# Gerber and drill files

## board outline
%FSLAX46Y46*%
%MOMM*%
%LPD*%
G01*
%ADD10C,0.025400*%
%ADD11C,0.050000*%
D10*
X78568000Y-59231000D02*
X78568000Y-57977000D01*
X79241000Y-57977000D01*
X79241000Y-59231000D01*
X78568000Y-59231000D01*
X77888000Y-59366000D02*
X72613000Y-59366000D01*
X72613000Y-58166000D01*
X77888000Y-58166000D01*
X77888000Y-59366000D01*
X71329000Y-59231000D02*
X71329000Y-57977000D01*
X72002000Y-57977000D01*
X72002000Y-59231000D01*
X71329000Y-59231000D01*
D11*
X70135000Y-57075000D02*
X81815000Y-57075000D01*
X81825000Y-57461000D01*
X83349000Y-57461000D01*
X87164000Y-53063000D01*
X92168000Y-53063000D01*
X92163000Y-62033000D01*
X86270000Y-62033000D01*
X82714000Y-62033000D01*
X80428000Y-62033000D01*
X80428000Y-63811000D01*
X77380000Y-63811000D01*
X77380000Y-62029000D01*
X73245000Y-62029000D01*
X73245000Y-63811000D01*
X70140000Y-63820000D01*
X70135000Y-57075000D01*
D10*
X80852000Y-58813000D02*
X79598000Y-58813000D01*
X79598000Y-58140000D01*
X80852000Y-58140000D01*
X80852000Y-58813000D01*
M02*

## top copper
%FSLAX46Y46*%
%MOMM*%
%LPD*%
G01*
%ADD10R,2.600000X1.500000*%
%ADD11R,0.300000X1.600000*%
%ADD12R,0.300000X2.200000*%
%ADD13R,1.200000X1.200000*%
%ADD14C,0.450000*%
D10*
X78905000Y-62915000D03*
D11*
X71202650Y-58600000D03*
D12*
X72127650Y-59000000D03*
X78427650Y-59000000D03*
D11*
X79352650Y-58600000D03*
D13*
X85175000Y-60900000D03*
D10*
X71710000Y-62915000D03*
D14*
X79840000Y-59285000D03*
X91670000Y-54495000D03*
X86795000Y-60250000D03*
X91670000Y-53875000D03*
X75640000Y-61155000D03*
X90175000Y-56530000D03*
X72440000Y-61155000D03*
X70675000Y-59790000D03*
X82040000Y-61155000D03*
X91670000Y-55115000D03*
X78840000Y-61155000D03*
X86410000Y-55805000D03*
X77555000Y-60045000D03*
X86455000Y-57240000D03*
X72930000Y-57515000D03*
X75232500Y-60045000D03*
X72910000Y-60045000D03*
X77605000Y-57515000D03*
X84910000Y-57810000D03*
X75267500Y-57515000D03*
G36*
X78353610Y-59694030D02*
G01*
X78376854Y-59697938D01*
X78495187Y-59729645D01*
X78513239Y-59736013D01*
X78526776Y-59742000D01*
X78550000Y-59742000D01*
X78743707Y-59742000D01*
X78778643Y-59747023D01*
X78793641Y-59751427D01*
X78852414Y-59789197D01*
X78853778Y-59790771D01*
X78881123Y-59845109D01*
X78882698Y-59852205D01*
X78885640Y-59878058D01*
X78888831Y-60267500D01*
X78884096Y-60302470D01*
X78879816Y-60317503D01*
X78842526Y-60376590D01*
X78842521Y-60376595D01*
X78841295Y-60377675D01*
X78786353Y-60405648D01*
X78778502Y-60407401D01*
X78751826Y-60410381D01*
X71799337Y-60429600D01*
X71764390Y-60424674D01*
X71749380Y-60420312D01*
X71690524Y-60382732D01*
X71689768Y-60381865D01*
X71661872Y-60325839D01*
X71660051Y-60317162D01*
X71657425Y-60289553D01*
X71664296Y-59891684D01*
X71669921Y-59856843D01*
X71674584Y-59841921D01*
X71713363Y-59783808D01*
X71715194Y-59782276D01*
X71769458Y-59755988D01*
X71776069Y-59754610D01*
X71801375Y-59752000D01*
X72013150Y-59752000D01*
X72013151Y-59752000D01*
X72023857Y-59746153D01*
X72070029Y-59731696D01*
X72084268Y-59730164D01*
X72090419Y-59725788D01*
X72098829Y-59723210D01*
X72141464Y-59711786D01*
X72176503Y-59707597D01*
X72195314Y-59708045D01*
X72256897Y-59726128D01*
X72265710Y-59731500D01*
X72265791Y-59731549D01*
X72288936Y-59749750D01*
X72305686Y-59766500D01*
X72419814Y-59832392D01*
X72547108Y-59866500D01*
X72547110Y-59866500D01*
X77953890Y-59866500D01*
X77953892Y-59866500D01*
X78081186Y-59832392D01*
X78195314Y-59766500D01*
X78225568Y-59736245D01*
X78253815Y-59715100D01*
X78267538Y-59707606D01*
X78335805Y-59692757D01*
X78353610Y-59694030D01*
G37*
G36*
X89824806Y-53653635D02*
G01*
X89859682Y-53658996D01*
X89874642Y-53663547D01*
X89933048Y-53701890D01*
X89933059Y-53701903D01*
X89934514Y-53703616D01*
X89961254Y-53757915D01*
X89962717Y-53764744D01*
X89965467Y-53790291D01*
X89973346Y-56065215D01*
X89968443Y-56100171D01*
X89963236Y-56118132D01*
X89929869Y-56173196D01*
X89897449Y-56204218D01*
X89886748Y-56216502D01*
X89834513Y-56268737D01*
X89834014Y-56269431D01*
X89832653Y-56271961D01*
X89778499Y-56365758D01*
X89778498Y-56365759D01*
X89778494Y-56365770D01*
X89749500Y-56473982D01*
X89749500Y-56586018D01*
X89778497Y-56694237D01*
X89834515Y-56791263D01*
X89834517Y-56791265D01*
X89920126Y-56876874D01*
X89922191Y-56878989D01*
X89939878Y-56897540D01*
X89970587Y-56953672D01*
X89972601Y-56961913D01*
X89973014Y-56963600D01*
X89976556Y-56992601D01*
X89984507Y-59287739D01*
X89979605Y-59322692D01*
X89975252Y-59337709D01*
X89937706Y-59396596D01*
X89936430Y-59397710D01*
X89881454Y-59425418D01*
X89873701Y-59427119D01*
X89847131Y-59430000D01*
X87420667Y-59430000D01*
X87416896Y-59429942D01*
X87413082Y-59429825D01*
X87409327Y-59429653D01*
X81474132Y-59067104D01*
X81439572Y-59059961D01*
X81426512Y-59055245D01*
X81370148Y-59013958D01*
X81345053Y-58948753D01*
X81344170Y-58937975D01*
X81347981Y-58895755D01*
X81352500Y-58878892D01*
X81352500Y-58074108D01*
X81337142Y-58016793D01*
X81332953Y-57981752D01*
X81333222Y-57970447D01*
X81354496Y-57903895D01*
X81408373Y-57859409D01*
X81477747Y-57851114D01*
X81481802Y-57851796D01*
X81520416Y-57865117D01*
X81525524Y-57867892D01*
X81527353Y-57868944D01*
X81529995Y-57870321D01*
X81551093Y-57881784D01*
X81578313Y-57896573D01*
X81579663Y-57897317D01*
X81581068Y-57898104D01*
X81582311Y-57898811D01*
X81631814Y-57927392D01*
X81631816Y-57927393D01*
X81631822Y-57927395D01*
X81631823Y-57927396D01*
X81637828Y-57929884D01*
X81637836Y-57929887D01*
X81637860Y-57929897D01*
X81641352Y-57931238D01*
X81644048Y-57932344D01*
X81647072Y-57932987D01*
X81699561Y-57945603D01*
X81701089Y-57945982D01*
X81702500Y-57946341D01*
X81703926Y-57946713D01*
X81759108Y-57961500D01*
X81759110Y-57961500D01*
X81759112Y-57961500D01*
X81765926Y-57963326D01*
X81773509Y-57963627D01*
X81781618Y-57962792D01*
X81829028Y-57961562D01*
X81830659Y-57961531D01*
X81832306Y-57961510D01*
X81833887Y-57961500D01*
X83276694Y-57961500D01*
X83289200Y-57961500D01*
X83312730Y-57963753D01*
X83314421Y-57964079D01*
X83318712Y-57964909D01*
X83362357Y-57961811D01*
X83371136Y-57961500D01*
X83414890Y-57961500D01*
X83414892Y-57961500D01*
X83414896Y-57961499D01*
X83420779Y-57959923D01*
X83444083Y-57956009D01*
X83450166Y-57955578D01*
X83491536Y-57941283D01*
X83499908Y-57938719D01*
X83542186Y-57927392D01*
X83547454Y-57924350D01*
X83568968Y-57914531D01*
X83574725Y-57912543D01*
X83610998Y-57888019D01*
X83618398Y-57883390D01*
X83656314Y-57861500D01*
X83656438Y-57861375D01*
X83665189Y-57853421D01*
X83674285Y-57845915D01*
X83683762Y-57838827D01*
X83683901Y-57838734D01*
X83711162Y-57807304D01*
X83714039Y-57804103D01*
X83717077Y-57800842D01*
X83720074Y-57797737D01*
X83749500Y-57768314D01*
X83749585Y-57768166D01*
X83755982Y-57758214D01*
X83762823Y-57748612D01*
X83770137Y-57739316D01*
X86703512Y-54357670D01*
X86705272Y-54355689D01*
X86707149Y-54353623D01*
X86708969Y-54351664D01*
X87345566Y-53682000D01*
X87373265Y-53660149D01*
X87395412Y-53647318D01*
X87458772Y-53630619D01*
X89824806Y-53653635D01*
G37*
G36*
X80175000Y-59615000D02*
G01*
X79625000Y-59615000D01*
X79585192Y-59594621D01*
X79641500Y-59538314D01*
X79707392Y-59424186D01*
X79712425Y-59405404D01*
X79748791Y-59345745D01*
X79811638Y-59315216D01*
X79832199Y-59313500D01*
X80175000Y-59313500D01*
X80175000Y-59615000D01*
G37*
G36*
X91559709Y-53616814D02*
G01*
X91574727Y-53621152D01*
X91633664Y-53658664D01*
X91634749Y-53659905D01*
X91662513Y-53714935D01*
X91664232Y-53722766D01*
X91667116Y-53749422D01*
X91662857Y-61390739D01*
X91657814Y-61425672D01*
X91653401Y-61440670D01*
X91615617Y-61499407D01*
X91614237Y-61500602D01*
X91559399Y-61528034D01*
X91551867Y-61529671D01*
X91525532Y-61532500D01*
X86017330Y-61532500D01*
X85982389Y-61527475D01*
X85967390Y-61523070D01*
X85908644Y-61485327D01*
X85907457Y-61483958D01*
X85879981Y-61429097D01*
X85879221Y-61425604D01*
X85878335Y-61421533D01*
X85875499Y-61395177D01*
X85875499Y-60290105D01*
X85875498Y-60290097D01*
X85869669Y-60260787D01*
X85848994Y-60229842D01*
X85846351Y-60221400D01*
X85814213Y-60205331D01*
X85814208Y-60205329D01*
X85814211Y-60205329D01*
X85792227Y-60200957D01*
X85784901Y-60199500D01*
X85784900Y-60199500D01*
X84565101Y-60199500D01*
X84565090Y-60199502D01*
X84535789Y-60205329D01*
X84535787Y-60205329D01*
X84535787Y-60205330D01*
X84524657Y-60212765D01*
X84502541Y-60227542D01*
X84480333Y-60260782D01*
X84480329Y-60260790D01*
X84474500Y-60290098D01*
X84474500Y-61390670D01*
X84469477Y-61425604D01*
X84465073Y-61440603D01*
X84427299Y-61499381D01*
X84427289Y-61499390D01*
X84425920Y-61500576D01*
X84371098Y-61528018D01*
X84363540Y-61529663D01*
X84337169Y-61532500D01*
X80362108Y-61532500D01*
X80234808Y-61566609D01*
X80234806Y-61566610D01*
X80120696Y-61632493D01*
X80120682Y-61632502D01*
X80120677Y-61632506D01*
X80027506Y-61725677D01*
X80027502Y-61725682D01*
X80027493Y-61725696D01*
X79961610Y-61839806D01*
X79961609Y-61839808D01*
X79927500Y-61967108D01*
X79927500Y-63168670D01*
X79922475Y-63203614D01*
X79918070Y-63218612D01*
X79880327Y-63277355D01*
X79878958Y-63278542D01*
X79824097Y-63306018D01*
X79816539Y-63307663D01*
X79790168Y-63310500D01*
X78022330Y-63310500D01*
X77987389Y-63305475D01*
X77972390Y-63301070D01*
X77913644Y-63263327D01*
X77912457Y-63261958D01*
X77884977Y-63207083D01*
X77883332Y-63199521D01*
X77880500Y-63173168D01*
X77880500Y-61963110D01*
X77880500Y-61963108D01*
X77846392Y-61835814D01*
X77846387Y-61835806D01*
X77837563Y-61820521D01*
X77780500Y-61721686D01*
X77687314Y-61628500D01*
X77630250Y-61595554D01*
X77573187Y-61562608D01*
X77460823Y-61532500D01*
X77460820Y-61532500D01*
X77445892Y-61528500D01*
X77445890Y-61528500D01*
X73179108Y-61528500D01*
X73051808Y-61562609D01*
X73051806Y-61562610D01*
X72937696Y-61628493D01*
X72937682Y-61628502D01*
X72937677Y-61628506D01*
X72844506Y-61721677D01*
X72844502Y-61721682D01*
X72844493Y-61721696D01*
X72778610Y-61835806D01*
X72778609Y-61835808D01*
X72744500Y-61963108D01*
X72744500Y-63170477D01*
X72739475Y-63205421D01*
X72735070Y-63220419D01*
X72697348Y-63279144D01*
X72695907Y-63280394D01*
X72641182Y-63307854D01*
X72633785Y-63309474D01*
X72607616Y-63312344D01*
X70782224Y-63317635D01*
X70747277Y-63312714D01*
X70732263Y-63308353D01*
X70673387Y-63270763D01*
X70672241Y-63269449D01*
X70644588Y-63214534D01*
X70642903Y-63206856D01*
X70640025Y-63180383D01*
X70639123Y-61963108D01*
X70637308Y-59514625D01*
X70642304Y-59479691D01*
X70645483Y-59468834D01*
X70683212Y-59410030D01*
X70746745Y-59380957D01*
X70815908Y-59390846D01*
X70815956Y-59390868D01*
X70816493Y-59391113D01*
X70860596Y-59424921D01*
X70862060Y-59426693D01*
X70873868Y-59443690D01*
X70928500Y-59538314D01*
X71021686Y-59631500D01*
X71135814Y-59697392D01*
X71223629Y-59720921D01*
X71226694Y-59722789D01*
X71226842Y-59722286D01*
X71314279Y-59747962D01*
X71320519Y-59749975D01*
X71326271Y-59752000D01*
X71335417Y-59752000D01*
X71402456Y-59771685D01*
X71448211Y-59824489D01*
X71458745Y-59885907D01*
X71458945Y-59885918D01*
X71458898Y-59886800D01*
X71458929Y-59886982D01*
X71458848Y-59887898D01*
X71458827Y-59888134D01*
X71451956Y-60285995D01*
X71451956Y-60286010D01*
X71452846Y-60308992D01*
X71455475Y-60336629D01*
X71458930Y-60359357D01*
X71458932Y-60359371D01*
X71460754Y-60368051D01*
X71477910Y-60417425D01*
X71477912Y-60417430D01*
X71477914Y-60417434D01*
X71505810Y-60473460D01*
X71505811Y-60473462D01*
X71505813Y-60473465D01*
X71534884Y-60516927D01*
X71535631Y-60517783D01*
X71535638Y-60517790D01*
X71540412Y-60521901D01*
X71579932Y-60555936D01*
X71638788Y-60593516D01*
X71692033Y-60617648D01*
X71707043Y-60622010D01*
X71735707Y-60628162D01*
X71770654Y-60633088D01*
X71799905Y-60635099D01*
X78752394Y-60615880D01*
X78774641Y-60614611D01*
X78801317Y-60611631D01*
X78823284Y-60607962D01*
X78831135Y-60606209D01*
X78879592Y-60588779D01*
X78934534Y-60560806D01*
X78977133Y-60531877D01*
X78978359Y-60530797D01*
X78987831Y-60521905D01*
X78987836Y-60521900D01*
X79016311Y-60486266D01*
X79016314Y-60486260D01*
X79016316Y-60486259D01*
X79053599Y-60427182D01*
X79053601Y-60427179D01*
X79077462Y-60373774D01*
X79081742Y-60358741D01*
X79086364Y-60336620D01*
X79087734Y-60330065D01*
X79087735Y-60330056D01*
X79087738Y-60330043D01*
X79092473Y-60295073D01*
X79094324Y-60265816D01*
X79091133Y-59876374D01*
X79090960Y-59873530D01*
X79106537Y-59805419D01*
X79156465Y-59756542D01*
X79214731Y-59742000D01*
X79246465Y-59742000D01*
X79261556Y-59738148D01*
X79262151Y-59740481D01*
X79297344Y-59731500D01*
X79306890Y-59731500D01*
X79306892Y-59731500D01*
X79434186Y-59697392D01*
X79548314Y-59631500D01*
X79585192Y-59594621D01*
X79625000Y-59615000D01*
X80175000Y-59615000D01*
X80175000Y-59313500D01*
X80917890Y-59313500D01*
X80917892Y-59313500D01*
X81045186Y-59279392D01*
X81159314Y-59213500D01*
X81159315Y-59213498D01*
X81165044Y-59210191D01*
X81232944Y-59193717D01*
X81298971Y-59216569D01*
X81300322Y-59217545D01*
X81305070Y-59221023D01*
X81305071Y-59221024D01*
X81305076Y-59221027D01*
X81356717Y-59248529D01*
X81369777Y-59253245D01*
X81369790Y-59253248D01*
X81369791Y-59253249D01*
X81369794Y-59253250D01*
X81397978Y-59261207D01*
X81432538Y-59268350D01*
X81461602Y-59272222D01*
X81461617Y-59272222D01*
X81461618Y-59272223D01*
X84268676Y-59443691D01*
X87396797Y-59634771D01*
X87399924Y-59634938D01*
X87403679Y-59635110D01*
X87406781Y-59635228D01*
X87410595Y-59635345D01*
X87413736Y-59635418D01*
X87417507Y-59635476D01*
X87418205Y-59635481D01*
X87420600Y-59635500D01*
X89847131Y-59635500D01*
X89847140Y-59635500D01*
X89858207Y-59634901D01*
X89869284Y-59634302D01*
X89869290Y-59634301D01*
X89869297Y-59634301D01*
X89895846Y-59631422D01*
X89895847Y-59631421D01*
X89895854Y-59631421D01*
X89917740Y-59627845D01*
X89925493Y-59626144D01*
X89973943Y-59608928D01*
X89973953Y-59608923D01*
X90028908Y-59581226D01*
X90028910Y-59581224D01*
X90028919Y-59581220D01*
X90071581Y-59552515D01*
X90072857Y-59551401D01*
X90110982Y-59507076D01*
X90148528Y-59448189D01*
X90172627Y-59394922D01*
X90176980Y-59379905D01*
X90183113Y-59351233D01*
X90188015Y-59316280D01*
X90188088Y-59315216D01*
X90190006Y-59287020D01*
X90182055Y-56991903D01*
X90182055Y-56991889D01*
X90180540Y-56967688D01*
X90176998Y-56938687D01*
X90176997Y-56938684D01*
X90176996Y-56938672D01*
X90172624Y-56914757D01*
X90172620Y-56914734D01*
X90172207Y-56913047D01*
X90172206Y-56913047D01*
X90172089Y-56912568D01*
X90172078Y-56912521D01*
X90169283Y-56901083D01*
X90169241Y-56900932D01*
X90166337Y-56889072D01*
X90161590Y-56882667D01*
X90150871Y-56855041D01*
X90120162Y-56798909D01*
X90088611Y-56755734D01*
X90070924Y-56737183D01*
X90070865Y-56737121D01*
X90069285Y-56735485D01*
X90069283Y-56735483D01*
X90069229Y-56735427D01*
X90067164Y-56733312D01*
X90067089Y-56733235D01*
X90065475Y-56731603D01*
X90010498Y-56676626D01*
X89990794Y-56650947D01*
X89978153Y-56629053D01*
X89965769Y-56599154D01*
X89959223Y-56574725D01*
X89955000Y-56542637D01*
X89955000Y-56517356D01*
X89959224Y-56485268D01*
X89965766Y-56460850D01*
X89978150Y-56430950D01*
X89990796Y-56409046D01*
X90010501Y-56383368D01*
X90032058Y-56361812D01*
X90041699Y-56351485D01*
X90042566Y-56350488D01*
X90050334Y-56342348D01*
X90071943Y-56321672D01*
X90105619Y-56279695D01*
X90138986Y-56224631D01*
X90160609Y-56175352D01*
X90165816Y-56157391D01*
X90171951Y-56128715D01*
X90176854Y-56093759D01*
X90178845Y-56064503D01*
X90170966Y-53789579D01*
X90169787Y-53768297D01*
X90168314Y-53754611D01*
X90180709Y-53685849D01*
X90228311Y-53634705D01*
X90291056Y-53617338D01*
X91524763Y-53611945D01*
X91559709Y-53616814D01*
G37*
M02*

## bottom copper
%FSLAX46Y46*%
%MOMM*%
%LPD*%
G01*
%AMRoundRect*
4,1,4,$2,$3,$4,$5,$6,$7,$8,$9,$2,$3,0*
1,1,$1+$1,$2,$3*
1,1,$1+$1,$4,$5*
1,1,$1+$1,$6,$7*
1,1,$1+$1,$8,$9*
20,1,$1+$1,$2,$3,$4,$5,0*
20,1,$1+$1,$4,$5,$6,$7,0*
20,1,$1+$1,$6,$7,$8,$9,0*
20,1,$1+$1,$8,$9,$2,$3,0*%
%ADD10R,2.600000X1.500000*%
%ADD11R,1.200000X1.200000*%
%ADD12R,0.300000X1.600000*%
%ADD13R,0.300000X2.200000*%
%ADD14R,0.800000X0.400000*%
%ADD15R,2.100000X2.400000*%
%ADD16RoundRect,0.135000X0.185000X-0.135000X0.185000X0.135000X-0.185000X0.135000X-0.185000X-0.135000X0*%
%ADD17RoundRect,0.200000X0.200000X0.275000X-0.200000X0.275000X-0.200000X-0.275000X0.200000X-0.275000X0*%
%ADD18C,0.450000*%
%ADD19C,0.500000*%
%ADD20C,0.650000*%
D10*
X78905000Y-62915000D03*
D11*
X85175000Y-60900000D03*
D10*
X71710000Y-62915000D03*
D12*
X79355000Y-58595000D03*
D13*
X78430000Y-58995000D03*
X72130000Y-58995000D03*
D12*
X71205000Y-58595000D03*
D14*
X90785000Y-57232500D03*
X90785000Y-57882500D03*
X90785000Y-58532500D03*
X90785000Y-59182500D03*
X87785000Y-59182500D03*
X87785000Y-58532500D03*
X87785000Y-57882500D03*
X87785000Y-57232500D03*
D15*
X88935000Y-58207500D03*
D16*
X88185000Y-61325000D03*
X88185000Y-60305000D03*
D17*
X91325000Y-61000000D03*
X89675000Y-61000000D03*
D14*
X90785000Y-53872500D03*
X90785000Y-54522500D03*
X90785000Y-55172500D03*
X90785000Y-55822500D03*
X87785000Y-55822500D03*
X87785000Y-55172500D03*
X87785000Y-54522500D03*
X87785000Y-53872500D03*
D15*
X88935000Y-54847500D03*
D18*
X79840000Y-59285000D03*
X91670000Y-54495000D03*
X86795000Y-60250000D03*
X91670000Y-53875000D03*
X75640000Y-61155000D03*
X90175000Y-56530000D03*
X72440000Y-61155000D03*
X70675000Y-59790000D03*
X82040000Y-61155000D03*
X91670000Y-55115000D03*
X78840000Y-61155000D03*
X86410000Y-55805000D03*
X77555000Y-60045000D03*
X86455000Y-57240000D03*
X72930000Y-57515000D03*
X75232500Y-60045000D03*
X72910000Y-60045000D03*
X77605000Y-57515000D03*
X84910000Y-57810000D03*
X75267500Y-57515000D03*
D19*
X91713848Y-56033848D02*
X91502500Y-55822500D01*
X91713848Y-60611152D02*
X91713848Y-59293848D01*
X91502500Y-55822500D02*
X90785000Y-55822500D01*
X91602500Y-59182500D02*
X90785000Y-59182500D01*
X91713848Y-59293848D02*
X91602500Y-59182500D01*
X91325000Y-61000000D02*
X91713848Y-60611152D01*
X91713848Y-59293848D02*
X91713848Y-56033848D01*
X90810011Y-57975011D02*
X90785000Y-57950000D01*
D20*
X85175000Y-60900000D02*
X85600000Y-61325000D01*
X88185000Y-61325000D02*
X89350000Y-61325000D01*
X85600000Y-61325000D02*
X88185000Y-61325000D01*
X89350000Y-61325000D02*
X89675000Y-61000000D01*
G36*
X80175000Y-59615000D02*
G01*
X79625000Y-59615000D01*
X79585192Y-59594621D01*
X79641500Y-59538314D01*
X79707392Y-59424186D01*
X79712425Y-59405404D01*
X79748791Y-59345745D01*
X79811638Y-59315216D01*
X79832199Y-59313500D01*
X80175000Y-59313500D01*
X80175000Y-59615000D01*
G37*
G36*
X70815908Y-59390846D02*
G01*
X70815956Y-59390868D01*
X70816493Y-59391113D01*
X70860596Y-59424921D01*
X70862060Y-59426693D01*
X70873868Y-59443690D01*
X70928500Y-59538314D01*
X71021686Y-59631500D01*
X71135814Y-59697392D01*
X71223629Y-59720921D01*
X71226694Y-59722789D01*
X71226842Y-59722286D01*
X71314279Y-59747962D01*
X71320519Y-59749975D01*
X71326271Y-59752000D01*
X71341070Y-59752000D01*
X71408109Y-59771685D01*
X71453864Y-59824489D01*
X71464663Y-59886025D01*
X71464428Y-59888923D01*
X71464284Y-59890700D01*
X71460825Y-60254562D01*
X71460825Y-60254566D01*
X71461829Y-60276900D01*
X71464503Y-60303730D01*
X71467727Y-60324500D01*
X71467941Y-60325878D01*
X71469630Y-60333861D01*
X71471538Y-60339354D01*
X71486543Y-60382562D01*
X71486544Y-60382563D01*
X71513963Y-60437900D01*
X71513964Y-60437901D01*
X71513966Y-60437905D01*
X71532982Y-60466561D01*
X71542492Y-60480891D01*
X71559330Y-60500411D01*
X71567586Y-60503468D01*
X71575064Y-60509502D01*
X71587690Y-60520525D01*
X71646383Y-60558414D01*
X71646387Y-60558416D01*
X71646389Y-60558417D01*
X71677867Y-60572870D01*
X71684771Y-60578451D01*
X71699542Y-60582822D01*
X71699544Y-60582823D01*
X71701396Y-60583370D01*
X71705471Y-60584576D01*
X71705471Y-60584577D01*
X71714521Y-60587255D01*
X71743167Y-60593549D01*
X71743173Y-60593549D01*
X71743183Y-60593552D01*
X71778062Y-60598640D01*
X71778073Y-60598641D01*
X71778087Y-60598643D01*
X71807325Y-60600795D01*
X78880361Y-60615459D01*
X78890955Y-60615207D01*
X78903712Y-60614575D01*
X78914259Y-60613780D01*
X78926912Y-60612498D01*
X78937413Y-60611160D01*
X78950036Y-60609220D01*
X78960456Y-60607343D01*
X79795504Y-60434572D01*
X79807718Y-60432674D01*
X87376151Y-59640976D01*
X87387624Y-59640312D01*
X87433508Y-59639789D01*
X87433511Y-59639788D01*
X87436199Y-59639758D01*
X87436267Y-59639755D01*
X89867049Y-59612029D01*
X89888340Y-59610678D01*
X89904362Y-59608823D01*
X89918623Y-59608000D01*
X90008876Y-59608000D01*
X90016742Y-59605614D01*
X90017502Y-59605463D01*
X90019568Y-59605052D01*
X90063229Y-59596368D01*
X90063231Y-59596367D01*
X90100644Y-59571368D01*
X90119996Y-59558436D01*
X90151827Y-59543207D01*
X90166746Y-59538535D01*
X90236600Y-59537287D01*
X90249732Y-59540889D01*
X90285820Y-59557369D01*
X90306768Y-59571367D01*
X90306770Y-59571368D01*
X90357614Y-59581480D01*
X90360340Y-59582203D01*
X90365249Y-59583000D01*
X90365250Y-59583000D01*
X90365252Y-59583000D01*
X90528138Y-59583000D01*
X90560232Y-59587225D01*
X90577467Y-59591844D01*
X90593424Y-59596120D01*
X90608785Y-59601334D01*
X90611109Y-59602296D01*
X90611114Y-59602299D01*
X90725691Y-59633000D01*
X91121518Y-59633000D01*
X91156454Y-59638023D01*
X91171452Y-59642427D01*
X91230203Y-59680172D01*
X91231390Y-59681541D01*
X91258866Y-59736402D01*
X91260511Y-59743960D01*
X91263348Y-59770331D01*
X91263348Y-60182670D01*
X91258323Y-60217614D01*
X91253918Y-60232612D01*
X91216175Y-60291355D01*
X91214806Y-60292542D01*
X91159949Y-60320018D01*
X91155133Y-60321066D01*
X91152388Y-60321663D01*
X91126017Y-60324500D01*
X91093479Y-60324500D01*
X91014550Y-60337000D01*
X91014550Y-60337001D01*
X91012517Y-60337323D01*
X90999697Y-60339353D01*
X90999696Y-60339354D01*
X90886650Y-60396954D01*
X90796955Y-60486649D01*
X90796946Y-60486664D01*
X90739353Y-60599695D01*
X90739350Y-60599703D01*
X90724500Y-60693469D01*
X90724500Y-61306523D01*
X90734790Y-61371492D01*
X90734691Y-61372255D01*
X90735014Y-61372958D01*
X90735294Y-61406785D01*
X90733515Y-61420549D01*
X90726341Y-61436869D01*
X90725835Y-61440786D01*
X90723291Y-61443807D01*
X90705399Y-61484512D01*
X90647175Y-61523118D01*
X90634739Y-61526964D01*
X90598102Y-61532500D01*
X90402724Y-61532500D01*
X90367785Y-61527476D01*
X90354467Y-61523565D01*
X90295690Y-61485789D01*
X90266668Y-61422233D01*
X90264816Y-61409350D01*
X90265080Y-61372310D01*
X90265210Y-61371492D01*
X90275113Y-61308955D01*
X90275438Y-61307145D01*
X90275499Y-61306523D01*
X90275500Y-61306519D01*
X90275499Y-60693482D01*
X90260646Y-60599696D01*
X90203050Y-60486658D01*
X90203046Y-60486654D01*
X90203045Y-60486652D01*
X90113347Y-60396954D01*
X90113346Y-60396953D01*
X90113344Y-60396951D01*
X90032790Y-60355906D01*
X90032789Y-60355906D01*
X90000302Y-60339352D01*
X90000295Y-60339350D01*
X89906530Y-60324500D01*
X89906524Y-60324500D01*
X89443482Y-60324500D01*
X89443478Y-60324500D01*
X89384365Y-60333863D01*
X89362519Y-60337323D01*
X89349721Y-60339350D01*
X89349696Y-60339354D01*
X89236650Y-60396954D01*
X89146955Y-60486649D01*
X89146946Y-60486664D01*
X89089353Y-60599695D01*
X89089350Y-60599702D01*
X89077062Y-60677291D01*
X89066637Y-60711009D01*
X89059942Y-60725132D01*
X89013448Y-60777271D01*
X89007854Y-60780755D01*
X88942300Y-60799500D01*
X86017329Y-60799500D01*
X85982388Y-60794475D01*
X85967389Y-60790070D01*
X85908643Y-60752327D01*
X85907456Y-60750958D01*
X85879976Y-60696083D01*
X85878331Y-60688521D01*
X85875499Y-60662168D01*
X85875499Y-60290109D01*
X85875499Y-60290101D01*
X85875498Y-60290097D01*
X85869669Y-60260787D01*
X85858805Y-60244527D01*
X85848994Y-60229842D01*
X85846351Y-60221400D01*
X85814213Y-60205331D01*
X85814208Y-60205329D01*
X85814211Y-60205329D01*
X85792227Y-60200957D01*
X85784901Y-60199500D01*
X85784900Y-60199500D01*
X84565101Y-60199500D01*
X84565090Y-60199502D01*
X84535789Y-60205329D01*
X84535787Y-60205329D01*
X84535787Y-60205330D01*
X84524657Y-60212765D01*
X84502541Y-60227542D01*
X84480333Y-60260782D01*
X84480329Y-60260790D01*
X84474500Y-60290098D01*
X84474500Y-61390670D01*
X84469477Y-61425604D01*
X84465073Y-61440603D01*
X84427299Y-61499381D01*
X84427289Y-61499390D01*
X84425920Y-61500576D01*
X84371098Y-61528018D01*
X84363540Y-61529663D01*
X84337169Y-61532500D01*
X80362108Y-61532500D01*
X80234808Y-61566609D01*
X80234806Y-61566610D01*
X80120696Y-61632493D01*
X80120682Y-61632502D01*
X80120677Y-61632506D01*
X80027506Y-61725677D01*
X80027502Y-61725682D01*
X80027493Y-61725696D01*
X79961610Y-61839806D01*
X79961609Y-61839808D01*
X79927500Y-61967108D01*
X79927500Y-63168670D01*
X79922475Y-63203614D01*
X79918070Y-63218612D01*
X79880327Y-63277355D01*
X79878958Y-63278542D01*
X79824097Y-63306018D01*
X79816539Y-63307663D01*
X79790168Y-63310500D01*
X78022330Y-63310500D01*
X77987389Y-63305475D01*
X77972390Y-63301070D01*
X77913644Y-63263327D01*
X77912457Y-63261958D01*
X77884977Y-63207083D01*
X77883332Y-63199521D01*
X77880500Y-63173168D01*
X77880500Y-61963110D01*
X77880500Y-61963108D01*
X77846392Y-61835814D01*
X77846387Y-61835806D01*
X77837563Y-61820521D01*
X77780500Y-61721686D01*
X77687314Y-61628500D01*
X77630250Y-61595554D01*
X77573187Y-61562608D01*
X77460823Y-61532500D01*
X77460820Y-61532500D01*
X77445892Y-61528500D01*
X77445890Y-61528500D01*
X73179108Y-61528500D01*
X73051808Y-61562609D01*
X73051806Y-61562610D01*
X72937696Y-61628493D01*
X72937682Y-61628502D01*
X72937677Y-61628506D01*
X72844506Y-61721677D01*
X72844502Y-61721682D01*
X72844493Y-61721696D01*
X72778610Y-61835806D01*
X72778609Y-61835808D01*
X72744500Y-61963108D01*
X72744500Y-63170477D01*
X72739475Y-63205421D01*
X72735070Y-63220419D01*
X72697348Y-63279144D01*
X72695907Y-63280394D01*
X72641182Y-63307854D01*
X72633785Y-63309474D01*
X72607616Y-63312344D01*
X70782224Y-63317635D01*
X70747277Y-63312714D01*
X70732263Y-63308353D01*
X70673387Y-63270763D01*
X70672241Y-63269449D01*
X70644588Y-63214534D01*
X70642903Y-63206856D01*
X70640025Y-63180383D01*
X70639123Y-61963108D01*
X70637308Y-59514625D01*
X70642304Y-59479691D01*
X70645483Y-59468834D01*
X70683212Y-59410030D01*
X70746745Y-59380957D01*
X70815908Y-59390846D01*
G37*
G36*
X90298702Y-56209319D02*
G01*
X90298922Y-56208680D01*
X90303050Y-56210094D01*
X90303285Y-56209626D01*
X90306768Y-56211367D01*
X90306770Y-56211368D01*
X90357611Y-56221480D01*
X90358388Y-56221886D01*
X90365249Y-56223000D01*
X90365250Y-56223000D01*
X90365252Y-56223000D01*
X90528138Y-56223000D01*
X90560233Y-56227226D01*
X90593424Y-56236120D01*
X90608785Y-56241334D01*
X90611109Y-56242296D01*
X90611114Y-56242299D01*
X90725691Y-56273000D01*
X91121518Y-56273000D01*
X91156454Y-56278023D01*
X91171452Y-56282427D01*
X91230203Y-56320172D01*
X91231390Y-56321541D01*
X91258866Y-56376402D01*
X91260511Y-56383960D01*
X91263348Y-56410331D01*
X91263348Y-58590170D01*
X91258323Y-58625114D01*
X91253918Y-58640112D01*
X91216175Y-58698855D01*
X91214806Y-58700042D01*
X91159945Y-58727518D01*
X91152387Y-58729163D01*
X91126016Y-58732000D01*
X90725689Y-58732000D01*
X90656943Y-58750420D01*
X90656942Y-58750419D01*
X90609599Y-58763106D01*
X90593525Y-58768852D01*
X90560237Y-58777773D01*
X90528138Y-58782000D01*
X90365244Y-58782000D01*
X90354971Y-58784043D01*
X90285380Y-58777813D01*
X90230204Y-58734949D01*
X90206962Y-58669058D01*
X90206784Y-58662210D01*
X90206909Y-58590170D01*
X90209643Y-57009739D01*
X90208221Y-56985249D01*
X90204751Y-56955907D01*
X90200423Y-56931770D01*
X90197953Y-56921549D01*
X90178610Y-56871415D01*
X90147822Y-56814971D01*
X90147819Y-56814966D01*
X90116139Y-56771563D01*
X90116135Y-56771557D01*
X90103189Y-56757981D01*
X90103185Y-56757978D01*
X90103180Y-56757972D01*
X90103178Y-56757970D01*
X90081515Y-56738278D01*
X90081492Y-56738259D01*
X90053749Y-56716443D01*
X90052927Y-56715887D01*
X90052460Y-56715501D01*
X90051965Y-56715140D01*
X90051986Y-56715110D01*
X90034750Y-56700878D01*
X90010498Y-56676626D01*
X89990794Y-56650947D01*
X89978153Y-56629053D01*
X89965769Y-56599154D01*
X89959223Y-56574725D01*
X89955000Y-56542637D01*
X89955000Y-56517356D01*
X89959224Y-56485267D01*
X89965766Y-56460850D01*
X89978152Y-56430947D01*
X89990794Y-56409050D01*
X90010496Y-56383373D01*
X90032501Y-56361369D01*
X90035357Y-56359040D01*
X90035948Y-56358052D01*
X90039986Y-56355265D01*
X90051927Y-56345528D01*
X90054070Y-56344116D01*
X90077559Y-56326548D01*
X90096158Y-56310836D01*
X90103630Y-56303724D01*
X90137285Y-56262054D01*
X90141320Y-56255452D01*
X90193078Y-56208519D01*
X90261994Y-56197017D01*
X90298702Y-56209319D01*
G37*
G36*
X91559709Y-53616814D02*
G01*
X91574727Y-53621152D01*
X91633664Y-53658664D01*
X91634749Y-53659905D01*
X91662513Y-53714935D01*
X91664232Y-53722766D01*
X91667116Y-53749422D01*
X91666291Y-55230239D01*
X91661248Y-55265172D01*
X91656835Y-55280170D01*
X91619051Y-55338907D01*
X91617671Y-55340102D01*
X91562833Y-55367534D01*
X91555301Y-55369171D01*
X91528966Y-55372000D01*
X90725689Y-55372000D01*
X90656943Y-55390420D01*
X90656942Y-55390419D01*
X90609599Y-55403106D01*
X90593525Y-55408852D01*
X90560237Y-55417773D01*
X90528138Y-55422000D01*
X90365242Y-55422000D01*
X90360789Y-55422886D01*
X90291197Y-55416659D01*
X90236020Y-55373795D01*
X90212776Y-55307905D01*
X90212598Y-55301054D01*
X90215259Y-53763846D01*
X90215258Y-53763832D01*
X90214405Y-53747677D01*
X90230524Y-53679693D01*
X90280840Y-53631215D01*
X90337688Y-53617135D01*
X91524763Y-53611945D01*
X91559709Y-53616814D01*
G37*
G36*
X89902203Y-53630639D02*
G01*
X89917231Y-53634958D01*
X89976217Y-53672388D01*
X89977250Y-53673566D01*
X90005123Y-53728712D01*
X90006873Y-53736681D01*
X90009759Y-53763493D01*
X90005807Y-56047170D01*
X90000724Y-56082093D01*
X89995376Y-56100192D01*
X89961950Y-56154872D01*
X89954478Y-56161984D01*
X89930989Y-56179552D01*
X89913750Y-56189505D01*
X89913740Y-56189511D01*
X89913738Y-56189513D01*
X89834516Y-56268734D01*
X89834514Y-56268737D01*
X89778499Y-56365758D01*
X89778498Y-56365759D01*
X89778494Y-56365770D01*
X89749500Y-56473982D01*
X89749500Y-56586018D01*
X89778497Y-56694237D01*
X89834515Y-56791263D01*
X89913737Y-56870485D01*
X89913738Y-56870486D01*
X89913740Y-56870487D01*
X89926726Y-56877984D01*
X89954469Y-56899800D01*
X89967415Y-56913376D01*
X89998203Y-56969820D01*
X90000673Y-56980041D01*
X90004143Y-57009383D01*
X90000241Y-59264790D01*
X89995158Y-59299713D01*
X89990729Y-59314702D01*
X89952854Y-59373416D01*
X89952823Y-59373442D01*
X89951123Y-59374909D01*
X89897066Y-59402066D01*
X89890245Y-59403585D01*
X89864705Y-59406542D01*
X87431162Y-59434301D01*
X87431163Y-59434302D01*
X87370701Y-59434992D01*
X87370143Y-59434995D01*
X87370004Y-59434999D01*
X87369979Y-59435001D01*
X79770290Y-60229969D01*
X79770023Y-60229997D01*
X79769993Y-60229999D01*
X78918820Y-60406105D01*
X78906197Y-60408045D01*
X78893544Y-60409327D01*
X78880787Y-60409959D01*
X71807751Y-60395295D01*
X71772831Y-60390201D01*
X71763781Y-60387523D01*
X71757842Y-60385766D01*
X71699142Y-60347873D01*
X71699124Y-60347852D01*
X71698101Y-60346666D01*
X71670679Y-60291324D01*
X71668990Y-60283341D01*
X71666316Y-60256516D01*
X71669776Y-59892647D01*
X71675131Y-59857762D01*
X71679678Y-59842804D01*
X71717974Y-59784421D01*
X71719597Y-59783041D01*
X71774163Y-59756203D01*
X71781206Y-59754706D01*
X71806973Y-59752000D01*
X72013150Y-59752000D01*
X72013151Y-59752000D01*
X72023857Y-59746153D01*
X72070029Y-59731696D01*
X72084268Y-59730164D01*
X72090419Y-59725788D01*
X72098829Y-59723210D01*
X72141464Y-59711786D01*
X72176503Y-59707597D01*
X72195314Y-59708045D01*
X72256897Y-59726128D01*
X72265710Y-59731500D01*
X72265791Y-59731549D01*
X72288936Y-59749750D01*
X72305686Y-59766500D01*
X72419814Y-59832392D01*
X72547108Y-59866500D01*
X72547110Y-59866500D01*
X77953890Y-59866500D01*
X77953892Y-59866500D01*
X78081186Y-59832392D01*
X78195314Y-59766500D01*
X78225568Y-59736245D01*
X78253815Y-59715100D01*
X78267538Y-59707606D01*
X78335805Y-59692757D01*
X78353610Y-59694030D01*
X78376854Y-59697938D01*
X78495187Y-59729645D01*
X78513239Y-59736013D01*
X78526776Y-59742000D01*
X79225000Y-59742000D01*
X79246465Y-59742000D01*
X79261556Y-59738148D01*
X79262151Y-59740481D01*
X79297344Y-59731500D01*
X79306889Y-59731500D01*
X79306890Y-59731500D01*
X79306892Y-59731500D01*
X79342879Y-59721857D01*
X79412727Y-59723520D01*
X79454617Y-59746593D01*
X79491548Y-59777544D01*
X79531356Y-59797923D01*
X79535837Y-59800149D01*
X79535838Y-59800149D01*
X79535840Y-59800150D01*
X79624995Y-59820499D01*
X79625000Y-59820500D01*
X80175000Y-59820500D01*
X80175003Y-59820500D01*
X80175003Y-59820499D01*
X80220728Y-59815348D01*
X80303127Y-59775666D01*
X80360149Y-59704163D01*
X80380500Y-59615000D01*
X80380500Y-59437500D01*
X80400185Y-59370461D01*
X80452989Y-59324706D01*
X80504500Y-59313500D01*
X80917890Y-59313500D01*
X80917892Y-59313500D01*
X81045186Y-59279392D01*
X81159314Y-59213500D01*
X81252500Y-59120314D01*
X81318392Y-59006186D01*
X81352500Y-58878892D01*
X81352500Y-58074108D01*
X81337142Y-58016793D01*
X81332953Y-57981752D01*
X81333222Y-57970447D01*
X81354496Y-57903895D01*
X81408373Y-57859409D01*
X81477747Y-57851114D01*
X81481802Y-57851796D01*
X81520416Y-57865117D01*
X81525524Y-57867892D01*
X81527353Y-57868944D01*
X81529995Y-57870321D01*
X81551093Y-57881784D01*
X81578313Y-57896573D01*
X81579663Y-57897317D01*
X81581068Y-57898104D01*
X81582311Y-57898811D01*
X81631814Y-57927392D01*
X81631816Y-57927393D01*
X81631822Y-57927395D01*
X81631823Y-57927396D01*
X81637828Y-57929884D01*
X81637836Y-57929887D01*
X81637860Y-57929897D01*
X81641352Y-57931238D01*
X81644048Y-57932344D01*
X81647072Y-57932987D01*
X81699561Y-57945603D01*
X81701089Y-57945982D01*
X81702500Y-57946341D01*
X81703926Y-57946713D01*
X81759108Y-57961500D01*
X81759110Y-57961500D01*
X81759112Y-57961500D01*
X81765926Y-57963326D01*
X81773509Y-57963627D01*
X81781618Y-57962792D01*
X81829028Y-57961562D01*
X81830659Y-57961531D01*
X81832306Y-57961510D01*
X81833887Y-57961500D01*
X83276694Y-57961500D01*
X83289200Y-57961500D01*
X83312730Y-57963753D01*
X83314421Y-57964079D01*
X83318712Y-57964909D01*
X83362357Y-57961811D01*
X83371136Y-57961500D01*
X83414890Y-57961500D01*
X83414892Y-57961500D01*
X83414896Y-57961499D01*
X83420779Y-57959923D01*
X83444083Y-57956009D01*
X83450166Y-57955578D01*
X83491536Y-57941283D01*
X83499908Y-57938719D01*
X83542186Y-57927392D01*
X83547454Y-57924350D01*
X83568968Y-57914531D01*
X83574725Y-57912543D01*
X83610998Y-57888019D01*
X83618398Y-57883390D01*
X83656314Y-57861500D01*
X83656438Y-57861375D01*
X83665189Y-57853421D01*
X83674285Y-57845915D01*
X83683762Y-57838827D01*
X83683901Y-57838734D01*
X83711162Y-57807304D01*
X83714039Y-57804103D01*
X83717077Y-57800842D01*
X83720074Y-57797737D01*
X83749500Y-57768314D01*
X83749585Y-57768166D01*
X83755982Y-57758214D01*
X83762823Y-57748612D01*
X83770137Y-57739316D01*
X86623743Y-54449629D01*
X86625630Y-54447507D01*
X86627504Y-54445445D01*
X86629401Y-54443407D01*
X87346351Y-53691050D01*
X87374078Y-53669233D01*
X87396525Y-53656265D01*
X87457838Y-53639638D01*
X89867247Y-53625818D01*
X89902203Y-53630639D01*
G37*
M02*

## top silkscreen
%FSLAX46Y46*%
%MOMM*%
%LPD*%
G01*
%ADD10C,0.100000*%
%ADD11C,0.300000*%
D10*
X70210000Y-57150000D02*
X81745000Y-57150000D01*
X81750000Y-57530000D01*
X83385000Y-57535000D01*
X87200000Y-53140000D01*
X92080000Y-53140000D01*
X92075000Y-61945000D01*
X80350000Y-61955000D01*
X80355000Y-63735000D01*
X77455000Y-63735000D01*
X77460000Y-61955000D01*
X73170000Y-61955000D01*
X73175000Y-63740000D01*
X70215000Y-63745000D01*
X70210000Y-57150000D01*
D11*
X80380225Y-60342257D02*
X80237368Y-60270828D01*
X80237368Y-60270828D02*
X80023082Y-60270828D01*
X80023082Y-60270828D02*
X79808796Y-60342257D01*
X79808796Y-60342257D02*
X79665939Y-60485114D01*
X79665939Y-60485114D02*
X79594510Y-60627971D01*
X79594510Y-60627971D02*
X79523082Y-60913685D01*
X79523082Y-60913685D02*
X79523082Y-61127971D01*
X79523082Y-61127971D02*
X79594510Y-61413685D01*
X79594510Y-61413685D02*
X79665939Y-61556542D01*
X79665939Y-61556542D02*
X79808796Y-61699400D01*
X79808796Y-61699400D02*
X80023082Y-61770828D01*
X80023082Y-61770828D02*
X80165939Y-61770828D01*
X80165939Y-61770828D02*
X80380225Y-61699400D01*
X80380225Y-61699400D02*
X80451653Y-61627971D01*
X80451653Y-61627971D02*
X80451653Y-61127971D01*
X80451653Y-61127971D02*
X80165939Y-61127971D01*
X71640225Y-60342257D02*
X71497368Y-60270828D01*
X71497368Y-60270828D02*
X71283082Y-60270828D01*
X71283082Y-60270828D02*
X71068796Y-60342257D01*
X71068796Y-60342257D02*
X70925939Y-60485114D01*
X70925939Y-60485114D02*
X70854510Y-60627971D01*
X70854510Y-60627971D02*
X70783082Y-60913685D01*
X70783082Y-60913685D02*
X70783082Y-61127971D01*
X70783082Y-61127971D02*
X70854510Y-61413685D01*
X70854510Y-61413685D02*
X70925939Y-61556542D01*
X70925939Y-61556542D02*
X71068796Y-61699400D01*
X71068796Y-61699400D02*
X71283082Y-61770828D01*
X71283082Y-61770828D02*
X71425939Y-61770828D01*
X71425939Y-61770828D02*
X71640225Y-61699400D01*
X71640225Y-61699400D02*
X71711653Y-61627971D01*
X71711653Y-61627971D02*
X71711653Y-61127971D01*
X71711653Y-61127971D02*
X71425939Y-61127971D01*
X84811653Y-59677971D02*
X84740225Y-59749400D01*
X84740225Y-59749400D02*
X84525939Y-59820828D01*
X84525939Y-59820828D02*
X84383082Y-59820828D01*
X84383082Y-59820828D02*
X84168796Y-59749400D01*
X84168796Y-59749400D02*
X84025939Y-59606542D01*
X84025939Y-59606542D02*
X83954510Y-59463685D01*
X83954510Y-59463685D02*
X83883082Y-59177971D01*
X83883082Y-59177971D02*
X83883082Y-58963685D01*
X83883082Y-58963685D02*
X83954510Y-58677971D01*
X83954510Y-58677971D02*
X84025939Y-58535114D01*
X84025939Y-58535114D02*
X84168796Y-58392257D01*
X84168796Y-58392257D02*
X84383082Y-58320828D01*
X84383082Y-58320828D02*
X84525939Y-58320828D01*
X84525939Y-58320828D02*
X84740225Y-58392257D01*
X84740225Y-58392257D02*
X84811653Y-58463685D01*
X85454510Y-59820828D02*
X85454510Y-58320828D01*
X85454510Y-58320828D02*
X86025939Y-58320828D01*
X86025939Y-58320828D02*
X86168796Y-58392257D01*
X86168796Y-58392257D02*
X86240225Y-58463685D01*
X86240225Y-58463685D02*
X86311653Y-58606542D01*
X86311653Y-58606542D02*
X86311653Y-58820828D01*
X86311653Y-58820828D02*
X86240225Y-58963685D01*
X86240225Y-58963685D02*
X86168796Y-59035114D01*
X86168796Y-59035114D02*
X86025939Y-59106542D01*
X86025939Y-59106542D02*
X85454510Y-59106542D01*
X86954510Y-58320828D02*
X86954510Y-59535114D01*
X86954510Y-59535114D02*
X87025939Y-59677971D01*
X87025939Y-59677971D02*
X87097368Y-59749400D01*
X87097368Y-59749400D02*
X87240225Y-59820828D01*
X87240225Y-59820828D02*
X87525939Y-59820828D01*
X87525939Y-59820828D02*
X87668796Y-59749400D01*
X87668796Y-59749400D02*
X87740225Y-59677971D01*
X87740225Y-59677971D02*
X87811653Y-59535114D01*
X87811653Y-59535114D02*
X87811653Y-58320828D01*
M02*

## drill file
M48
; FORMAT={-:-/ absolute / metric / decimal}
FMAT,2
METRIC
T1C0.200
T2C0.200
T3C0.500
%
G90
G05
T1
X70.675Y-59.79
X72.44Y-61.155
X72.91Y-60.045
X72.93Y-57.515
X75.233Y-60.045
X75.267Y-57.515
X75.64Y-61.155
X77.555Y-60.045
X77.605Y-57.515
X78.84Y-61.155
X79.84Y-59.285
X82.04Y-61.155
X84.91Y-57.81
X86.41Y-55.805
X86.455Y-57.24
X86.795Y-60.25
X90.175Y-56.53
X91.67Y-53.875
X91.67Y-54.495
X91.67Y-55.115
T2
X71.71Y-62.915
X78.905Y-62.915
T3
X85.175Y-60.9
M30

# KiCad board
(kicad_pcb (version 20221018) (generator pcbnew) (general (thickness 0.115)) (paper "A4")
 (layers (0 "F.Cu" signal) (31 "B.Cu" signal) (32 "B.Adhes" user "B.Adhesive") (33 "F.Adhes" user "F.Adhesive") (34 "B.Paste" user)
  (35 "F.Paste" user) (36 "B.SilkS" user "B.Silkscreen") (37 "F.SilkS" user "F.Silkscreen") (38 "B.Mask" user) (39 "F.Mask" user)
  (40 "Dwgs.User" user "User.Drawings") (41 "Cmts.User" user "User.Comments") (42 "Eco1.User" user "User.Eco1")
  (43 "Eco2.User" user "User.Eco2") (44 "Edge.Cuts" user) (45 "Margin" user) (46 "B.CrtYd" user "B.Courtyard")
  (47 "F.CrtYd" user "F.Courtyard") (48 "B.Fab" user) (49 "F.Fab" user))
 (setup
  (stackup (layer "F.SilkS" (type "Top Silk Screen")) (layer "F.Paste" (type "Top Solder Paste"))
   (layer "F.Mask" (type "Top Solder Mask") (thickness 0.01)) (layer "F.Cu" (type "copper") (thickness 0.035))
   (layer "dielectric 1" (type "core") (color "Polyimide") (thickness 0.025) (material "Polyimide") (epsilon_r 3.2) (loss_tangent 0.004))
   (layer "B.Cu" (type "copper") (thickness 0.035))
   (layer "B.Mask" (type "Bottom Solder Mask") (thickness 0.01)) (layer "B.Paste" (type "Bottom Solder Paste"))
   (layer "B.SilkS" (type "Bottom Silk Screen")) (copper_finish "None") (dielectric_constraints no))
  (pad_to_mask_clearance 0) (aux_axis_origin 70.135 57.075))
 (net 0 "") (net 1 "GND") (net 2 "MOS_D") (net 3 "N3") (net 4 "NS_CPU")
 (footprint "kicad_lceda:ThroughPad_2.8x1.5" (layer "F.Cu") (at 78.905 62.915)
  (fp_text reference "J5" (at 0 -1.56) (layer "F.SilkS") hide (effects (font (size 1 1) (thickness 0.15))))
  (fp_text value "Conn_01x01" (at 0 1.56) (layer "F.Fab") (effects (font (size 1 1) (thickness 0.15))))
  (pad "1" thru_hole rect (at 0 0) (size 2.6 1.5) (drill 0.2) (layers "*.Cu" "*.Mask") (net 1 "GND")))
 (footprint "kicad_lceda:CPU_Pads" (layer "F.Cu") (at 75.07765 58.6)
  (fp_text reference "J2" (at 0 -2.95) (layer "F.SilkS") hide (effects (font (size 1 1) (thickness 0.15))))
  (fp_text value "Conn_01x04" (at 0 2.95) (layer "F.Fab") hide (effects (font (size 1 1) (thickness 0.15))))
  (pad "1" smd rect (at -3.875 0) (size 0.3 1.6) (layers "F.Cu" "F.Mask") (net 1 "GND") (zone_connect 2))
  (pad "2" smd rect (at -2.95 1) (size 0.3 2.2) (drill (offset 0 -0.6)) (layers "F.Cu" "F.Mask") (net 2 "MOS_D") (clearance 0.3)
   (zone_connect 2))
  (pad "3" smd rect (at 3.35 1) (size 0.3 2.2) (drill (offset 0 -0.6)) (layers "F.Cu" "F.Mask") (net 2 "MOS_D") (clearance 0.3)
   (zone_connect 2))
  (pad "4" smd rect (at 4.275 0) (size 0.3 1.6) (layers "F.Cu" "F.Mask") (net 1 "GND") (zone_connect 2)))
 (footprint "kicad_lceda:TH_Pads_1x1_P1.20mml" (layer "F.Cu") (at 85.175 60.9)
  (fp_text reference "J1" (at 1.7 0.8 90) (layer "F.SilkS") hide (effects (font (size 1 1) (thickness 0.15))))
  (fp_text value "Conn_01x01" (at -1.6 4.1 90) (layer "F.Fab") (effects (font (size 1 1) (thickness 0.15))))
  (pad "1" thru_hole rect (at 0 0) (size 1.2 1.2) (drill 0.5) (layers "*.Cu" "*.Mask") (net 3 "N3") (clearance 0.1) (zone_connect 2)))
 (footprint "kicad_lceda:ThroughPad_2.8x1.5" (layer "F.Cu") (at 71.71 62.915)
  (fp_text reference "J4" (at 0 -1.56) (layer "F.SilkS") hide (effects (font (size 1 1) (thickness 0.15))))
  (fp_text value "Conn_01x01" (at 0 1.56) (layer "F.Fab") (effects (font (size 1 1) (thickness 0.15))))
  (pad "1" thru_hole rect (at 0 0) (size 2.6 1.5) (drill 0.2) (layers "*.Cu" "*.Mask") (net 1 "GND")))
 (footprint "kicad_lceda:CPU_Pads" (layer "B.Cu") (at 75.48 58.595 180)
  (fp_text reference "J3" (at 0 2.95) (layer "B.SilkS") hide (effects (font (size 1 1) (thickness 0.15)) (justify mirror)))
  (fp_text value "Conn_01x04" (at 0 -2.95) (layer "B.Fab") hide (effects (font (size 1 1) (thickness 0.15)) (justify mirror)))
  (pad "1" smd rect (at -3.875 0 180) (size 0.3 1.6) (layers "B.Cu" "B.Mask") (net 1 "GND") (zone_connect 2))
  (pad "2" smd rect (at -2.95 -1 180) (size 0.3 2.2) (drill (offset 0 0.6)) (layers "B.Cu" "B.Mask") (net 2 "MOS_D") (clearance 0.3)
   (zone_connect 2))
  (pad "3" smd rect (at 3.35 -1 180) (size 0.3 2.2) (drill (offset 0 0.6)) (layers "B.Cu" "B.Mask") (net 2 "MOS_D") (clearance 0.3)
   (zone_connect 2))
  (pad "4" smd rect (at 4.275 0 180) (size 0.3 1.6) (layers "B.Cu" "B.Mask") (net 1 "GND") (zone_connect 2)))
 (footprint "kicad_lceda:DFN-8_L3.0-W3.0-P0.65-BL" (layer "B.Cu") (at 89.285 58.2075 -90)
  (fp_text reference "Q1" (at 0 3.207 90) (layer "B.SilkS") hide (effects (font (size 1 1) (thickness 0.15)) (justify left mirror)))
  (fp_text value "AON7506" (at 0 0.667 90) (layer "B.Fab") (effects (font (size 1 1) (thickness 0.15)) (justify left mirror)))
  (pad "1" smd rect (at -0.975 -1.5 90) (size 0.4 0.8) (layers "B.Cu" "B.Paste" "B.Mask") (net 1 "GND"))
  (pad "2" smd rect (at -0.325 -1.5 90) (size 0.4 0.8) (layers "B.Cu" "B.Paste" "B.Mask") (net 1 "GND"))
  (pad "3" smd rect (at 0.325 -1.5 90) (size 0.4 0.8) (layers "B.Cu" "B.Paste" "B.Mask") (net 1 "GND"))
  (pad "4" smd rect (at 0.975 -1.5 90) (size 0.4 0.8) (layers "B.Cu" "B.Paste" "B.Mask") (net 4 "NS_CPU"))
  (pad "5" smd rect (at 0.975 1.5 90) (size 0.4 0.8) (layers "B.Cu" "B.Paste" "B.Mask") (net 2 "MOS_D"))
  (pad "6" smd rect (at 0.325 1.5 90) (size 0.4 0.8) (layers "B.Cu" "B.Paste" "B.Mask") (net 2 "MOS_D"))
  (pad "7" smd rect (at -0.325 1.5 90) (size 0.4 0.8) (layers "B.Cu" "B.Paste" "B.Mask") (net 2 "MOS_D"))
  (pad "8" smd rect (at -0.975 1.5 90) (size 0.4 0.8) (layers "B.Cu" "B.Paste" "B.Mask") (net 2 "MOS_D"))
  (pad "9" smd rect (at 0 0.35 270) (size 2.4 2.1) (layers "B.Cu" "B.Paste" "B.Mask") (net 2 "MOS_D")))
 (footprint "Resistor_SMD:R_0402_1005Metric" (layer "B.Cu") (at 88.185 60.815 90)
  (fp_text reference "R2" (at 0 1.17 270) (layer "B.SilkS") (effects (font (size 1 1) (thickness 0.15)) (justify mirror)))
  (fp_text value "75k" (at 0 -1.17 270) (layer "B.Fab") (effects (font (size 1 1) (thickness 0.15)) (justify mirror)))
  (pad "1" smd roundrect (at -0.51 0 90) (size 0.54 0.64) (layers "B.Cu" "B.Paste" "B.Mask") (roundrect_rratio 0.25) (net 3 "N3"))
  (pad "2" smd roundrect (at 0.51 0 90) (size 0.54 0.64) (layers "B.Cu" "B.Paste" "B.Mask") (roundrect_rratio 0.25) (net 1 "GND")))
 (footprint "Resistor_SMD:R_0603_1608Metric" (layer "B.Cu") (at 90.5 61 180)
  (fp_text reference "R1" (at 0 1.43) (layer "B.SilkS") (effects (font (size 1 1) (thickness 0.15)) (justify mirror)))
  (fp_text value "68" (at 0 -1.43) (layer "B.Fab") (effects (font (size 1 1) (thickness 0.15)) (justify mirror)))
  (pad "1" smd roundrect (at -0.825 0 180) (size 0.8 0.95) (layers "B.Cu" "B.Paste" "B.Mask") (roundrect_rratio 0.25) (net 4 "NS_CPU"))
  (pad "2" smd roundrect (at 0.825 0 180) (size 0.8 0.95) (layers "B.Cu" "B.Paste" "B.Mask") (roundrect_rratio 0.25) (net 3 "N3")))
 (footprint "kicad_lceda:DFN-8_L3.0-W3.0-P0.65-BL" (layer "B.Cu") (at 89.285 54.8475 -90)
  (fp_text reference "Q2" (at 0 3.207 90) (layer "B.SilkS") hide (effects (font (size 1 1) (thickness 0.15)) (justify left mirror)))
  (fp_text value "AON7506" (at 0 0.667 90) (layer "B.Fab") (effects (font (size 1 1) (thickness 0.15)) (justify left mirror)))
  (pad "1" smd rect (at -0.975 -1.5 90) (size 0.4 0.8) (layers "B.Cu" "B.Paste" "B.Mask") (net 1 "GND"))
  (pad "2" smd rect (at -0.325 -1.5 90) (size 0.4 0.8) (layers "B.Cu" "B.Paste" "B.Mask") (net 1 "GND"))
  (pad "3" smd rect (at 0.325 -1.5 90) (size 0.4 0.8) (layers "B.Cu" "B.Paste" "B.Mask") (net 1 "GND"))
  (pad "4" smd rect (at 0.975 -1.5 90) (size 0.4 0.8) (layers "B.Cu" "B.Paste" "B.Mask") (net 4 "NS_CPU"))
  (pad "5" smd rect (at 0.975 1.5 90) (size 0.4 0.8) (layers "B.Cu" "B.Paste" "B.Mask") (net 2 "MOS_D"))
  (pad "6" smd rect (at 0.325 1.5 90) (size 0.4 0.8) (layers "B.Cu" "B.Paste" "B.Mask") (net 2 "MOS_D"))
  (pad "7" smd rect (at -0.325 1.5 90) (size 0.4 0.8) (layers "B.Cu" "B.Paste" "B.Mask") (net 2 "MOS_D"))
  (pad "8" smd rect (at -0.975 1.5 90) (size 0.4 0.8) (layers "B.Cu" "B.Paste" "B.Mask") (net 2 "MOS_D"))
  (pad "9" smd rect (at 0 0.35 270) (size 2.4 2.1) (layers "B.Cu" "B.Paste" "B.Mask") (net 2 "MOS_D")))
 (gr_poly
  (pts (xy 70.21 57.15) (xy 81.745 57.15) (xy 81.75 57.53) (xy 83.385 57.535) (xy 87.2 53.14) (xy 92.08 53.14) (xy 92.075 61.945)
   (xy 80.35 61.955) (xy 80.355 63.735) (xy 77.455 63.735) (xy 77.46 61.955) (xy 73.17 61.955) (xy 73.175 63.74) (xy 70.215 63.745))
  (stroke (width 0.1) (type solid)) (fill none) (layer "F.SilkS"))
 (gr_poly
  (pts (xy 78.568 59.231) (xy 78.568 57.977) (xy 79.241 57.977) (xy 79.241 59.231)) (stroke (width 0.0254) (type solid)) (fill none)
  (layer "Edge.Cuts"))
 (gr_poly
  (pts (xy 77.888 59.366) (xy 72.613 59.366) (xy 72.613 58.166) (xy 77.888 58.166)) (stroke (width 0.0254) (type solid)) (fill none)
  (layer "Edge.Cuts"))
 (gr_poly
  (pts (xy 71.329 59.231) (xy 71.329 57.977) (xy 72.002 57.977) (xy 72.002 59.231)) (stroke (width 0.0254) (type solid)) (fill none)
  (layer "Edge.Cuts"))
 (gr_poly
  (pts (xy 70.135 57.075) (xy 81.815 57.075) (xy 81.825 57.461) (xy 83.349 57.461) (xy 87.164 53.063) (xy 92.168 53.063) (xy 92.163 62.033)
   (xy 86.27 62.033) (xy 82.714 62.033) (xy 80.428 62.033) (xy 80.428 63.811) (xy 77.38 63.811) (xy 77.38 62.029) (xy 73.245 62.029)
   (xy 73.245 63.811) (xy 70.14 63.82))
  (stroke (width 0.05) (type solid)) (fill none) (layer "Edge.Cuts"))
 (gr_poly
  (pts (xy 80.852 58.813) (xy 79.598 58.813) (xy 79.598 58.14) (xy 80.852 58.14)) (stroke (width 0.0254) (type solid)) (fill none)
  (layer "Edge.Cuts"))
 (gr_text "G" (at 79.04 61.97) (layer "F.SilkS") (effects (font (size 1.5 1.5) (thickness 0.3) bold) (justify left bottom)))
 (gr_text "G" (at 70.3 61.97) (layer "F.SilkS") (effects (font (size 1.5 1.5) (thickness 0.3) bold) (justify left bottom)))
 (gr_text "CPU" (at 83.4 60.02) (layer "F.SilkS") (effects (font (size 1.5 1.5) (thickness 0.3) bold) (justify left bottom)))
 (segment (start 91.713848 56.033848) (end 91.5025 55.8225) (width 0.5) (layer "B.Cu") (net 4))
 (segment (start 91.713848 60.611152) (end 91.713848 59.293848) (width 0.5) (layer "B.Cu") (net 4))
 (segment (start 91.5025 55.8225) (end 90.785 55.8225) (width 0.5) (layer "B.Cu") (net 4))
 (segment (start 91.6025 59.1825) (end 90.785 59.1825) (width 0.5) (layer "B.Cu") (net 4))
 (segment (start 91.713848 59.293848) (end 91.6025 59.1825) (width 0.5) (layer "B.Cu") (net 4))
 (segment (start 91.325 61) (end 91.713848 60.611152) (width 0.5) (layer "B.Cu") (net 4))
 (segment (start 91.713848 59.293848) (end 91.713848 56.033848) (width 0.5) (layer "B.Cu") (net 4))
 (via (at 79.84 59.285) (size 0.45) (drill 0.2) (layers "F.Cu" "B.Cu") (free) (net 1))
 (via (at 91.67 54.495) (size 0.45) (drill 0.2) (layers "F.Cu" "B.Cu") (free) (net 1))
 (via (at 86.795 60.25) (size 0.45) (drill 0.2) (layers "F.Cu" "B.Cu") (free) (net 1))
 (via (at 91.67 53.875) (size 0.45) (drill 0.2) (layers "F.Cu" "B.Cu") (free) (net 1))
 (via (at 75.64 61.155) (size 0.45) (drill 0.2) (layers "F.Cu" "B.Cu") (free) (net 1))
 (via (at 90.175 56.53) (size 0.45) (drill 0.2) (layers "F.Cu" "B.Cu") (free) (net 1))
 (via (at 72.44 61.155) (size 0.45) (drill 0.2) (layers "F.Cu" "B.Cu") (free) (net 1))
 (via (at 70.675 59.79) (size 0.45) (drill 0.2) (layers "F.Cu" "B.Cu") (free) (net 1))
 (via (at 82.04 61.155) (size 0.45) (drill 0.2) (layers "F.Cu" "B.Cu") (free) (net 1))
 (via (at 91.67 55.115) (size 0.45) (drill 0.2) (layers "F.Cu" "B.Cu") (free) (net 1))
 (via (at 78.84 61.155) (size 0.45) (drill 0.2) (layers "F.Cu" "B.Cu") (free) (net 1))
 (segment (start 90.810011 57.975011) (end 90.785 57.95) (width 0.5) (layer "B.Cu") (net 1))
 (via (at 86.41 55.805) (size 0.45) (drill 0.2) (layers "F.Cu" "B.Cu") (free) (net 2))
 (via (at 77.555 60.045) (size 0.45) (drill 0.2) (layers "F.Cu" "B.Cu") (free) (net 2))
 (via (at 86.455 57.24) (size 0.45) (drill 0.2) (layers "F.Cu" "B.Cu") (free) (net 2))
 (via (at 72.93 57.515) (size 0.45) (drill 0.2) (layers "F.Cu" "B.Cu") (free) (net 2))
 (via (at 75.2325 60.045) (size 0.45) (drill 0.2) (layers "F.Cu" "B.Cu") (free) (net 2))
 (via (at 72.91 60.045) (size 0.45) (drill 0.2) (layers "F.Cu" "B.Cu") (free) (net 2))
 (via (at 77.605 57.515) (size 0.45) (drill 0.2) (layers "F.Cu" "B.Cu") (free) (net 2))
 (via (at 84.91 57.81) (size 0.45) (drill 0.2) (layers "F.Cu" "B.Cu") (free) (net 2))
 (via (at 75.2675 57.515) (size 0.45) (drill 0.2) (layers "F.Cu" "B.Cu") (free) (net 2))
 (segment (start 85.175 60.9) (end 85.6 61.325) (width 0.65) (layer "B.Cu") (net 3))
 (segment (start 88.185 61.325) (end 89.35 61.325) (width 0.65) (layer "B.Cu") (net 3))
 (segment (start 85.6 61.325) (end 88.185 61.325) (width 0.65) (layer "B.Cu") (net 3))
 (segment (start 89.35 61.325) (end 89.675 61) (width 0.65) (layer "B.Cu") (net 3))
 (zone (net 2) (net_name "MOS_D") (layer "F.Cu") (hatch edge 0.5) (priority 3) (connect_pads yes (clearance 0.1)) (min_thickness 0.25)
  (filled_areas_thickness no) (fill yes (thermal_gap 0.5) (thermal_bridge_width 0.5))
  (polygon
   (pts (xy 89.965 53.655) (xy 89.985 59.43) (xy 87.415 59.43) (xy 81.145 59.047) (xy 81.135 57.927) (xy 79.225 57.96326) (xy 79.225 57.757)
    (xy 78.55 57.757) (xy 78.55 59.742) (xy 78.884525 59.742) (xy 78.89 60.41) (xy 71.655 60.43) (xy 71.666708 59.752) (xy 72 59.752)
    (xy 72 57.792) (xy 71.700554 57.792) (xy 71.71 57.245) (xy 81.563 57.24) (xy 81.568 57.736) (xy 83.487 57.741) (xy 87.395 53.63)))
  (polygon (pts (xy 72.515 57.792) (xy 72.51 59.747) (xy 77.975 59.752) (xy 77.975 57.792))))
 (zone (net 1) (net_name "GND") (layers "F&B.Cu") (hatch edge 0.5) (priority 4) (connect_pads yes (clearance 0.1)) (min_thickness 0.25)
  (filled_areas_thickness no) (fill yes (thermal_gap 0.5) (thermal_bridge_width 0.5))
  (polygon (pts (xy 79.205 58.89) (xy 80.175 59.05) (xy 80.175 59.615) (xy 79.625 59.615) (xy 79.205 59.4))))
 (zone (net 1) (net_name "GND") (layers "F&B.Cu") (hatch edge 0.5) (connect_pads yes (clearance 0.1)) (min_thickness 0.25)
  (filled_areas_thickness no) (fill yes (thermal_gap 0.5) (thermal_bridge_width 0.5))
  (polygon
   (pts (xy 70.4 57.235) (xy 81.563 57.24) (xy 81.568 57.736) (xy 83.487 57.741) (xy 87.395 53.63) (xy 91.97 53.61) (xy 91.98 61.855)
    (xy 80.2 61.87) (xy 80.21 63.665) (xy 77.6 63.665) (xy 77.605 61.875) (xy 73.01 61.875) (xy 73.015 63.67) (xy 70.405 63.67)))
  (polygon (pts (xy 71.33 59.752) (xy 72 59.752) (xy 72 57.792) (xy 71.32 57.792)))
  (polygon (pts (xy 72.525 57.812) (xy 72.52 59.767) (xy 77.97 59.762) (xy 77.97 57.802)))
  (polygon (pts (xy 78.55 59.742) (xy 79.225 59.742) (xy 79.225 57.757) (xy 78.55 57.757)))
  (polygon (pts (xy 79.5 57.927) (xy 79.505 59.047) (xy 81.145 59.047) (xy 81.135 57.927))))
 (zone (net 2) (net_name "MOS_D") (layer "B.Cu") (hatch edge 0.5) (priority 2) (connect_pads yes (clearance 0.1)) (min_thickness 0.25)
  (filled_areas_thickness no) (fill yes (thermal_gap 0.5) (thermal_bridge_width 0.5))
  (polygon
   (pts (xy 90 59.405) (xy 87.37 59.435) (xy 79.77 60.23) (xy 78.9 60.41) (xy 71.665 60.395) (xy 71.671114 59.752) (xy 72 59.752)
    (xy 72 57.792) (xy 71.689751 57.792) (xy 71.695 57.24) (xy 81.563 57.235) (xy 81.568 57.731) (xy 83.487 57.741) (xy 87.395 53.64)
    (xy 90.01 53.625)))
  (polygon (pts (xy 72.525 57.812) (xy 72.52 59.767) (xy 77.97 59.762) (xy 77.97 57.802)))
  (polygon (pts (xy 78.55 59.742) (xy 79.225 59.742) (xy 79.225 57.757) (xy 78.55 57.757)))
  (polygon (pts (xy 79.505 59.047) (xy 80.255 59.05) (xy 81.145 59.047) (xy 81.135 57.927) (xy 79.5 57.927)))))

